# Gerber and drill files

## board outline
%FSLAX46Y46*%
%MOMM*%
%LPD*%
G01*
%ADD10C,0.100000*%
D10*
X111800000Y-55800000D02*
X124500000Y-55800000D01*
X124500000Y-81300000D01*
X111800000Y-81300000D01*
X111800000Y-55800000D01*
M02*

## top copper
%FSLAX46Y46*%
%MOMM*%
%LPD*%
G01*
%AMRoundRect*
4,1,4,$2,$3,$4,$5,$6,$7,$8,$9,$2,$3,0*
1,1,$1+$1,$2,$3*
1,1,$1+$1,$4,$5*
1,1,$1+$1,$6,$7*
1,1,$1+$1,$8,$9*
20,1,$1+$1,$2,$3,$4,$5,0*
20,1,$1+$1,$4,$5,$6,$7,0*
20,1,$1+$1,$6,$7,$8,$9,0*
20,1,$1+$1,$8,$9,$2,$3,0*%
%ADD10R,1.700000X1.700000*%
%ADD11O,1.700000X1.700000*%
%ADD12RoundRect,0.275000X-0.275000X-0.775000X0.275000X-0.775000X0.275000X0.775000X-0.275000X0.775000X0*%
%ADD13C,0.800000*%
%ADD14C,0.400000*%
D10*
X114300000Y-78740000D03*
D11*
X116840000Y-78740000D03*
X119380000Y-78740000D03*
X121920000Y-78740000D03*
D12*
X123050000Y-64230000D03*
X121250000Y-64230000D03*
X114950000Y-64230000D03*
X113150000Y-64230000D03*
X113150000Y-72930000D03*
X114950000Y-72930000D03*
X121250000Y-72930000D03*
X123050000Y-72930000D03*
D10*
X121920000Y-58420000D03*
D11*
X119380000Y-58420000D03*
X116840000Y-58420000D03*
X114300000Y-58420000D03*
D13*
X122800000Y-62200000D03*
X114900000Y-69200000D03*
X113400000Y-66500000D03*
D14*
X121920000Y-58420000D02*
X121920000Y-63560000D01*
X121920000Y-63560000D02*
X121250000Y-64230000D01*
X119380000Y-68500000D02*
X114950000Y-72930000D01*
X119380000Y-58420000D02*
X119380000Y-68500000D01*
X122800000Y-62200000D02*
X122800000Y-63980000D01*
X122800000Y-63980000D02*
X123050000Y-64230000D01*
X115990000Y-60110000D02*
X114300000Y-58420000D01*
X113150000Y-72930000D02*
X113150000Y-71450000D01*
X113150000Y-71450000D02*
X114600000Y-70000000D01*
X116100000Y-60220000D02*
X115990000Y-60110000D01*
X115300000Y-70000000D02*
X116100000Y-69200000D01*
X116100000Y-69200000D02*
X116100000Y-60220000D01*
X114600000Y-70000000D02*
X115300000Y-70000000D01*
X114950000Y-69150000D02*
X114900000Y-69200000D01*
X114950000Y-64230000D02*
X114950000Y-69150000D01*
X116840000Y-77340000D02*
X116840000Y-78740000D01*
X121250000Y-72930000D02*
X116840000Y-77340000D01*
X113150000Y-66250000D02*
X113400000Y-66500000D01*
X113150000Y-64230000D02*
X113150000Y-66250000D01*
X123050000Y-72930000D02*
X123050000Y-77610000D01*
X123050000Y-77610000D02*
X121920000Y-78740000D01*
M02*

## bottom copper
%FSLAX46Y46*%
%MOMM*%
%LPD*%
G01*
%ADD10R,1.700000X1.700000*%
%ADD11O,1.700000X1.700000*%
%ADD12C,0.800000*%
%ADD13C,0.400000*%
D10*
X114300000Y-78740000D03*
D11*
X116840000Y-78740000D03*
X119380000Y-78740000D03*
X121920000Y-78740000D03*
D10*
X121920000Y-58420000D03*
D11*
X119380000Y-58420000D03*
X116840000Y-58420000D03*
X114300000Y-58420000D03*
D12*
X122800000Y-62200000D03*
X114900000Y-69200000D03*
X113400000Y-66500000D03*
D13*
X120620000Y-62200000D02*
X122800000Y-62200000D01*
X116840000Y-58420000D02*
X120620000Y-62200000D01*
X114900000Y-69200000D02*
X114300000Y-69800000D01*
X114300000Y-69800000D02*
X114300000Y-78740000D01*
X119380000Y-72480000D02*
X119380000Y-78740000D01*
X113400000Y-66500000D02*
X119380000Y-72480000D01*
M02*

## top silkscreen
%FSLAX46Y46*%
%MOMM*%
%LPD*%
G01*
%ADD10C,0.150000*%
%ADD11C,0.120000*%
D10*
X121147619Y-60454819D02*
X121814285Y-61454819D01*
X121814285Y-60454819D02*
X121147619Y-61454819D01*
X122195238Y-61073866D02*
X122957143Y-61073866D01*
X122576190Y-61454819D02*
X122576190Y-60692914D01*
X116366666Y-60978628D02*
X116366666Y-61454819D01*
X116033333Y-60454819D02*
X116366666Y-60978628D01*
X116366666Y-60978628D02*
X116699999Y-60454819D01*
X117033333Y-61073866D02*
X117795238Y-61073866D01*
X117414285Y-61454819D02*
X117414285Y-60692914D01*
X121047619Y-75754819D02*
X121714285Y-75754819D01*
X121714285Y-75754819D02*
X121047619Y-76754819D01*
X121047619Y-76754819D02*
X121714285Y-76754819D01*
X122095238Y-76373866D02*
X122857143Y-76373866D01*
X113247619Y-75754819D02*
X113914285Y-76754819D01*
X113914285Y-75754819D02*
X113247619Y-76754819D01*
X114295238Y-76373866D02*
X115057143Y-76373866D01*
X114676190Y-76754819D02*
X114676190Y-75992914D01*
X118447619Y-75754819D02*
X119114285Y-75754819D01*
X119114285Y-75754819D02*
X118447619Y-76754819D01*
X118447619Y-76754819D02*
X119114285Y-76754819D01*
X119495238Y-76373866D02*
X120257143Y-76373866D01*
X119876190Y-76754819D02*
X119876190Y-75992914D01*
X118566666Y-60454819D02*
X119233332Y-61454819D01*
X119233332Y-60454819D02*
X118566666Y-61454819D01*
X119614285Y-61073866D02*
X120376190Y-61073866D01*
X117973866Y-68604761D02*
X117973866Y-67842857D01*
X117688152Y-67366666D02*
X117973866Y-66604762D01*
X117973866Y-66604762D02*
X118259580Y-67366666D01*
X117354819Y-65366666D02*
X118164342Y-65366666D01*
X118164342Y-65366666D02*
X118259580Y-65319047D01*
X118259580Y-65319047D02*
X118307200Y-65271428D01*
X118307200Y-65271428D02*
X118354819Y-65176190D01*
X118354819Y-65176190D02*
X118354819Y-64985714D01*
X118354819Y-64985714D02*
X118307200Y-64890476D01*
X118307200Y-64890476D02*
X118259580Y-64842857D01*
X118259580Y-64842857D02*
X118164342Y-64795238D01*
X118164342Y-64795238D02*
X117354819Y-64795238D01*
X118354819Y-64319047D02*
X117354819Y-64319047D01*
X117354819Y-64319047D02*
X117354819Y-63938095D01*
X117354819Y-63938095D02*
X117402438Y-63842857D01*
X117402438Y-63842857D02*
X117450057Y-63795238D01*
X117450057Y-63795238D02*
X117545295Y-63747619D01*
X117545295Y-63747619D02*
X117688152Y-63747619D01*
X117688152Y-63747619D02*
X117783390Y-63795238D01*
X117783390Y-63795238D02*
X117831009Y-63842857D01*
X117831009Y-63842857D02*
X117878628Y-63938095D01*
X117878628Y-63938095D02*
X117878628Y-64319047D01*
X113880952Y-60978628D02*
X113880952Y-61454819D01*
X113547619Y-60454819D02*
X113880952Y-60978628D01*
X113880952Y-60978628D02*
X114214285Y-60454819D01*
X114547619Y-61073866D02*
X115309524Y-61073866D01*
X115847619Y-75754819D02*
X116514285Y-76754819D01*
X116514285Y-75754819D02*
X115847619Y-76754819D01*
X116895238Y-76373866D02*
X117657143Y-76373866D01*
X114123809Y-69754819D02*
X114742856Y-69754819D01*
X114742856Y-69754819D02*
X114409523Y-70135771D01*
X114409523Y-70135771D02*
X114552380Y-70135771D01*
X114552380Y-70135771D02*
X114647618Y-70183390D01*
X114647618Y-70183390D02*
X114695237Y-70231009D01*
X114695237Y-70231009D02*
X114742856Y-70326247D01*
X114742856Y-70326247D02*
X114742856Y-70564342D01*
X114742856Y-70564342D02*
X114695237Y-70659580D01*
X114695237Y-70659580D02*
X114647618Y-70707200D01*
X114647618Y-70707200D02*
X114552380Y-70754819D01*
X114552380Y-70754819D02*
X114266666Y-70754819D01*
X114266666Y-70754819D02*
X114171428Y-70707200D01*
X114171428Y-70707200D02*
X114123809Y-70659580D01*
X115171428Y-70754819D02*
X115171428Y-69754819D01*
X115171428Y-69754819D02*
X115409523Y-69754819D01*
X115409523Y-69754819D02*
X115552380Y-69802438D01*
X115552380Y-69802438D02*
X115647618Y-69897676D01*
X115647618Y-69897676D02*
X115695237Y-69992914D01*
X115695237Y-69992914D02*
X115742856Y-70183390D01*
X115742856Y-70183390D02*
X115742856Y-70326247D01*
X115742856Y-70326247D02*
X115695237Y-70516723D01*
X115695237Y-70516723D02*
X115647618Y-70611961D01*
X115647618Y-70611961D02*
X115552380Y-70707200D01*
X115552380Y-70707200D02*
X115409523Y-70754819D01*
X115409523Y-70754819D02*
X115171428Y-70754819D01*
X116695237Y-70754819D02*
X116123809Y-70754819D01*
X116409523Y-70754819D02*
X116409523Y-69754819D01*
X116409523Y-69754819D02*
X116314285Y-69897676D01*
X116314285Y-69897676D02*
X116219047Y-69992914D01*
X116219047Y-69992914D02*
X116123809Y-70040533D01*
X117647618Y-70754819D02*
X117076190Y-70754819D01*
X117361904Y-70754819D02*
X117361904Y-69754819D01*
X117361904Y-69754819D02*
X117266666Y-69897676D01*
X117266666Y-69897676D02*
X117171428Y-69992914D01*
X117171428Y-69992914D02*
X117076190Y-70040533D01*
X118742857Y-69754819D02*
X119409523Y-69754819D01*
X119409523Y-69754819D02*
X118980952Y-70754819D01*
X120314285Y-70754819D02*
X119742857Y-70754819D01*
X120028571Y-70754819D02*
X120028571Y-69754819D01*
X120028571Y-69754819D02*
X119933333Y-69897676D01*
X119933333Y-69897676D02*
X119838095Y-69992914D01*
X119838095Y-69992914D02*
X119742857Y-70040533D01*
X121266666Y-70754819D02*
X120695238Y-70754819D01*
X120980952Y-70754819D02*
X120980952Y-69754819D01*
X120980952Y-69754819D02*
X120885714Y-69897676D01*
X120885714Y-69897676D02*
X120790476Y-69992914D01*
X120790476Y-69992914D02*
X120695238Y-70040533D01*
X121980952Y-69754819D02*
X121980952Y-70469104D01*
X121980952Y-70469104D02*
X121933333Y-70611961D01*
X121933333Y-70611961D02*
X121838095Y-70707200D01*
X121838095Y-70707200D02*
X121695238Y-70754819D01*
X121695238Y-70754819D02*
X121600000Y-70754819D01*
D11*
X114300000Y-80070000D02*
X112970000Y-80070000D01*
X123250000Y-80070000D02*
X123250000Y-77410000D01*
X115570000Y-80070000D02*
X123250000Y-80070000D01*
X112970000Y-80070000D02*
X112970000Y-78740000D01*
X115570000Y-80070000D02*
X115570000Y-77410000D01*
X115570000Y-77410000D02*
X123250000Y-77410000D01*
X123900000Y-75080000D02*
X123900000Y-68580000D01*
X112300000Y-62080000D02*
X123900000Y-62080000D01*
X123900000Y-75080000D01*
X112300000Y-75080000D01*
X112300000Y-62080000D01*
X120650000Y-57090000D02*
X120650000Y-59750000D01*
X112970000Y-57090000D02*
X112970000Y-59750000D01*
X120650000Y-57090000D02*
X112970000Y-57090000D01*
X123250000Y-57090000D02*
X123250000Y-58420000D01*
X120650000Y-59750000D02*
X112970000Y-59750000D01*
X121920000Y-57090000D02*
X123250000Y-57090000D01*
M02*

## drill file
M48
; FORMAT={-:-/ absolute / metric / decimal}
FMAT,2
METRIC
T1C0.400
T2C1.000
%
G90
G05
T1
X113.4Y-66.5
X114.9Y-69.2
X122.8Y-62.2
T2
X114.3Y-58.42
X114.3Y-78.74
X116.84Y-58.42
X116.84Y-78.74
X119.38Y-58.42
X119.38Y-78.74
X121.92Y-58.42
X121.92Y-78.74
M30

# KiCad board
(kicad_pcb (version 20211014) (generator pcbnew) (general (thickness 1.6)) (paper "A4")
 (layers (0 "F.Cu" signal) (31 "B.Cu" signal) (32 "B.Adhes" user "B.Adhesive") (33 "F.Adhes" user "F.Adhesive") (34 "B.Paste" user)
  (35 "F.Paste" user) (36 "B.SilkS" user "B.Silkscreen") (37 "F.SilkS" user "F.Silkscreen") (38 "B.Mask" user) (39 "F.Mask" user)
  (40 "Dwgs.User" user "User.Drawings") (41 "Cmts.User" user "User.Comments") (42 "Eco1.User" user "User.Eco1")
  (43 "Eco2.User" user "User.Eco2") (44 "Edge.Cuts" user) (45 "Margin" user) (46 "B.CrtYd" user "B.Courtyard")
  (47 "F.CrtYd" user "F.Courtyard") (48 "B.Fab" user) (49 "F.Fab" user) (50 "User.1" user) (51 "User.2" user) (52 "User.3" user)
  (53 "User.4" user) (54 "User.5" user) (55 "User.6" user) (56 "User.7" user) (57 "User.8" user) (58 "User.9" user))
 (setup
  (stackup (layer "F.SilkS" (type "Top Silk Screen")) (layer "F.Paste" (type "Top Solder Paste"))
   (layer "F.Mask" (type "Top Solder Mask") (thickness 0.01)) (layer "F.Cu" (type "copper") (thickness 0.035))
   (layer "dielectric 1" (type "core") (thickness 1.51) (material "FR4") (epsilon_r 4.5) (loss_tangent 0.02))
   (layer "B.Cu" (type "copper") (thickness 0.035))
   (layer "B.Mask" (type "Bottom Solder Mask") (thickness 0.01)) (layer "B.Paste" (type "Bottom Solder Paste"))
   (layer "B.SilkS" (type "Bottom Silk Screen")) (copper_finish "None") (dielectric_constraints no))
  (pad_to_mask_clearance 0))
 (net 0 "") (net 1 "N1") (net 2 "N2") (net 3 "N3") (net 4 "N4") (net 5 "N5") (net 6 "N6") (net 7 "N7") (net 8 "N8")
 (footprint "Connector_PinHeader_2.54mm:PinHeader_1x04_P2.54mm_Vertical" (layer "F.Cu") (at 114.3 78.74 90)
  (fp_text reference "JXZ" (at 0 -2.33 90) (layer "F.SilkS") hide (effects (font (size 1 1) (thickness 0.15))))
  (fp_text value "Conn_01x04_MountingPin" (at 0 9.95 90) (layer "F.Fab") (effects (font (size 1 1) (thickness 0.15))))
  (fp_line (start -1.33 0) (end -1.33 -1.33) (layer "F.SilkS") (width 0.12))
  (fp_line (start -1.33 8.95) (end 1.33 8.95) (layer "F.SilkS") (width 0.12))
  (fp_line (start -1.33 1.27) (end -1.33 8.95) (layer "F.SilkS") (width 0.12))
  (fp_line (start -1.33 -1.33) (end 0 -1.33) (layer "F.SilkS") (width 0.12))
  (fp_line (start -1.33 1.27) (end 1.33 1.27) (layer "F.SilkS") (width 0.12))
  (fp_line (start 1.33 1.27) (end 1.33 8.95) (layer "F.SilkS") (width 0.12))
  (pad "1" thru_hole rect (at 0 0 90) (size 1.7 1.7) (drill 1) (layers *.Cu *.Mask) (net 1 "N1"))
  (pad "2" thru_hole oval (at 0 2.54 90) (size 1.7 1.7) (drill 1) (layers *.Cu *.Mask) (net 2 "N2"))
  (pad "3" thru_hole oval (at 0 5.08 90) (size 1.7 1.7) (drill 1) (layers *.Cu *.Mask) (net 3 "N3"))
  (pad "4" thru_hole oval (at 0 7.62 90) (size 1.7 1.7) (drill 1) (layers *.Cu *.Mask) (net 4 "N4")))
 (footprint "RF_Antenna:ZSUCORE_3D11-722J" (layer "F.Cu") (at 118.1 68.58)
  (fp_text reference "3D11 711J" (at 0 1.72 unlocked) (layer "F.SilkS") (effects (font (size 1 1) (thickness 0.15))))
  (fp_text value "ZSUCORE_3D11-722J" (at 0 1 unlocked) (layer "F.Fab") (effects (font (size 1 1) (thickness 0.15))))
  (fp_line (start 5.8 6.5) (end 5.8 0) (layer "F.SilkS") (width 0.12))
  (fp_rect (start -5.8 6.5) (end 5.8 -6.5) (layer "F.SilkS") (width 0.12) (fill none))
  (pad "1" smd roundrect (at 4.95 -4.35) (size 1.1 2.1) (layers "F.Cu" "F.Paste" "F.Mask") (roundrect_rratio 0.25) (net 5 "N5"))
  (pad "2" smd roundrect (at 3.15 -4.35) (size 1.1 2.1) (layers "F.Cu" "F.Paste" "F.Mask") (roundrect_rratio 0.25) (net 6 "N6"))
  (pad "3" smd roundrect (at -3.15 -4.35) (size 1.1 2.1) (layers "F.Cu" "F.Paste" "F.Mask") (roundrect_rratio 0.25) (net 1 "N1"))
  (pad "4" smd roundrect (at -4.95 -4.35) (size 1.1 2.1) (layers "F.Cu" "F.Paste" "F.Mask") (roundrect_rratio 0.25) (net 3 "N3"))
  (pad "5" smd roundrect (at -4.95 4.35) (size 1.1 2.1) (layers "F.Cu" "F.Paste" "F.Mask") (roundrect_rratio 0.25) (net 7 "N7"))
  (pad "6" smd roundrect (at -3.15 4.35) (size 1.1 2.1) (layers "F.Cu" "F.Paste" "F.Mask") (roundrect_rratio 0.25) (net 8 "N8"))
  (pad "7" smd roundrect (at 3.15 4.35) (size 1.1 2.1) (layers "F.Cu" "F.Paste" "F.Mask") (roundrect_rratio 0.25) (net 2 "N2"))
  (pad "8" smd roundrect (at 4.95 4.35) (size 1.1 2.1) (layers "F.Cu" "F.Paste" "F.Mask") (roundrect_rratio 0.25) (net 4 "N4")))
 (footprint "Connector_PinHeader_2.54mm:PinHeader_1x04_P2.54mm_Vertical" (layer "F.Cu") (at 121.92 58.42 -90)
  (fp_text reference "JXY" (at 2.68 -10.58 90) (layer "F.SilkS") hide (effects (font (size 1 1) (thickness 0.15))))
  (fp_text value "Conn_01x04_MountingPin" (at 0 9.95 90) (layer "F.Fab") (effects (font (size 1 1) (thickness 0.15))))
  (fp_line (start -1.33 1.27) (end 1.33 1.27) (layer "F.SilkS") (width 0.12))
  (fp_line (start -1.33 8.95) (end 1.33 8.95) (layer "F.SilkS") (width 0.12))
  (fp_line (start -1.33 1.27) (end -1.33 8.95) (layer "F.SilkS") (width 0.12))
  (fp_line (start -1.33 -1.33) (end 0 -1.33) (layer "F.SilkS") (width 0.12))
  (fp_line (start 1.33 1.27) (end 1.33 8.95) (layer "F.SilkS") (width 0.12))
  (fp_line (start -1.33 0) (end -1.33 -1.33) (layer "F.SilkS") (width 0.12))
  (pad "1" thru_hole rect (at 0 0 270) (size 1.7 1.7) (drill 1) (layers *.Cu *.Mask) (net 6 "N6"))
  (pad "2" thru_hole oval (at 0 2.54 270) (size 1.7 1.7) (drill 1) (layers *.Cu *.Mask) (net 8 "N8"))
  (pad "3" thru_hole oval (at 0 5.08 270) (size 1.7 1.7) (drill 1) (layers *.Cu *.Mask) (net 5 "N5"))
  (pad "4" thru_hole oval (at 0 7.62 270) (size 1.7 1.7) (drill 1) (layers *.Cu *.Mask) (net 7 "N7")))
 (gr_rect (start 111.8 55.8) (end 124.5 81.3) (layer "Edge.Cuts") (width 0.1) (fill none))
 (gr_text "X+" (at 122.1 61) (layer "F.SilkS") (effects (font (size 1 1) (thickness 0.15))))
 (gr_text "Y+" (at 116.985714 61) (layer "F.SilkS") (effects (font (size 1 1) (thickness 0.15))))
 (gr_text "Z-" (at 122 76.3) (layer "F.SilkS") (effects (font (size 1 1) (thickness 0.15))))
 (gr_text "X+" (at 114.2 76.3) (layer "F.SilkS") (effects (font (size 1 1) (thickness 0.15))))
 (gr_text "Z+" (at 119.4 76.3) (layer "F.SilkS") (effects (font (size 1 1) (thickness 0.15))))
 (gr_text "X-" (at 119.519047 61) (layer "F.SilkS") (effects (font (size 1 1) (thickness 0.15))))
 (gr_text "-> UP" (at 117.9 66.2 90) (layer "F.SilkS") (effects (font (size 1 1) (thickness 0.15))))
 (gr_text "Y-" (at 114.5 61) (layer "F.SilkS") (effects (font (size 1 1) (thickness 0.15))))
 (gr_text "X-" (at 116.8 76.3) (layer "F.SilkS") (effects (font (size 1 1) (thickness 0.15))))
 (segment (start 121.92 58.42) (end 121.92 63.56) (width 0.4) (layer "F.Cu") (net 6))
 (segment (start 121.92 63.56) (end 121.25 64.23) (width 0.4) (layer "F.Cu") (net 6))
 (segment (start 119.38 68.5) (end 114.95 72.93) (width 0.4) (layer "F.Cu") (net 8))
 (segment (start 119.38 58.42) (end 119.38 68.5) (width 0.4) (layer "F.Cu") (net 8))
 (segment (start 122.8 62.2) (end 122.8 63.98) (width 0.4) (layer "F.Cu") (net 5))
 (segment (start 122.8 63.98) (end 123.05 64.23) (width 0.4) (layer "F.Cu") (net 5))
 (via (at 122.8 62.2) (size 0.8) (drill 0.4) (layers "F.Cu" "B.Cu") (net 5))
 (segment (start 120.62 62.2) (end 122.8 62.2) (width 0.4) (layer "B.Cu") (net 5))
 (segment (start 116.84 58.42) (end 120.62 62.2) (width 0.4) (layer "B.Cu") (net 5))
 (segment (start 115.99 60.11) (end 114.3 58.42) (width 0.4) (layer "F.Cu") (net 7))
 (segment (start 113.15 72.93) (end 113.15 71.45) (width 0.4) (layer "F.Cu") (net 7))
 (segment (start 113.15 71.45) (end 114.6 70) (width 0.4) (layer "F.Cu") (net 7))
 (segment (start 116.1 60.22) (end 115.99 60.11) (width 0.4) (layer "F.Cu") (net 7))
 (segment (start 115.3 70) (end 116.1 69.2) (width 0.4) (layer "F.Cu") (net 7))
 (segment (start 116.1 69.2) (end 116.1 60.22) (width 0.4) (layer "F.Cu") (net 7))
 (segment (start 114.6 70) (end 115.3 70) (width 0.4) (layer "F.Cu") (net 7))
 (segment (start 114.95 69.15) (end 114.9 69.2) (width 0.4) (layer "F.Cu") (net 1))
 (segment (start 114.95 64.23) (end 114.95 69.15) (width 0.4) (layer "F.Cu") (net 1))
 (via (at 114.9 69.2) (size 0.8) (drill 0.4) (layers "F.Cu" "B.Cu") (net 1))
 (segment (start 114.9 69.2) (end 114.3 69.8) (width 0.4) (layer "B.Cu") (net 1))
 (segment (start 114.3 69.8) (end 114.3 78.74) (width 0.4) (layer "B.Cu") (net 1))
 (segment (start 116.84 77.34) (end 116.84 78.74) (width 0.4) (layer "F.Cu") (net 2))
 (segment (start 121.25 72.93) (end 116.84 77.34) (width 0.4) (layer "F.Cu") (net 2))
 (segment (start 113.15 66.25) (end 113.4 66.5) (width 0.4) (layer "F.Cu") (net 3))
 (segment (start 113.15 64.23) (end 113.15 66.25) (width 0.4) (layer "F.Cu") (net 3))
 (via (at 113.4 66.5) (size 0.8) (drill 0.4) (layers "F.Cu" "B.Cu") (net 3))
 (segment (start 119.38 72.48) (end 119.38 78.74) (width 0.4) (layer "B.Cu") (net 3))
 (segment (start 113.4 66.5) (end 119.38 72.48) (width 0.4) (layer "B.Cu") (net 3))
 (segment (start 123.05 72.93) (end 123.05 77.61) (width 0.4) (layer "F.Cu") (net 4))
 (segment (start 123.05 77.61) (end 121.92 78.74) (width 0.4) (layer "F.Cu") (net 4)))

